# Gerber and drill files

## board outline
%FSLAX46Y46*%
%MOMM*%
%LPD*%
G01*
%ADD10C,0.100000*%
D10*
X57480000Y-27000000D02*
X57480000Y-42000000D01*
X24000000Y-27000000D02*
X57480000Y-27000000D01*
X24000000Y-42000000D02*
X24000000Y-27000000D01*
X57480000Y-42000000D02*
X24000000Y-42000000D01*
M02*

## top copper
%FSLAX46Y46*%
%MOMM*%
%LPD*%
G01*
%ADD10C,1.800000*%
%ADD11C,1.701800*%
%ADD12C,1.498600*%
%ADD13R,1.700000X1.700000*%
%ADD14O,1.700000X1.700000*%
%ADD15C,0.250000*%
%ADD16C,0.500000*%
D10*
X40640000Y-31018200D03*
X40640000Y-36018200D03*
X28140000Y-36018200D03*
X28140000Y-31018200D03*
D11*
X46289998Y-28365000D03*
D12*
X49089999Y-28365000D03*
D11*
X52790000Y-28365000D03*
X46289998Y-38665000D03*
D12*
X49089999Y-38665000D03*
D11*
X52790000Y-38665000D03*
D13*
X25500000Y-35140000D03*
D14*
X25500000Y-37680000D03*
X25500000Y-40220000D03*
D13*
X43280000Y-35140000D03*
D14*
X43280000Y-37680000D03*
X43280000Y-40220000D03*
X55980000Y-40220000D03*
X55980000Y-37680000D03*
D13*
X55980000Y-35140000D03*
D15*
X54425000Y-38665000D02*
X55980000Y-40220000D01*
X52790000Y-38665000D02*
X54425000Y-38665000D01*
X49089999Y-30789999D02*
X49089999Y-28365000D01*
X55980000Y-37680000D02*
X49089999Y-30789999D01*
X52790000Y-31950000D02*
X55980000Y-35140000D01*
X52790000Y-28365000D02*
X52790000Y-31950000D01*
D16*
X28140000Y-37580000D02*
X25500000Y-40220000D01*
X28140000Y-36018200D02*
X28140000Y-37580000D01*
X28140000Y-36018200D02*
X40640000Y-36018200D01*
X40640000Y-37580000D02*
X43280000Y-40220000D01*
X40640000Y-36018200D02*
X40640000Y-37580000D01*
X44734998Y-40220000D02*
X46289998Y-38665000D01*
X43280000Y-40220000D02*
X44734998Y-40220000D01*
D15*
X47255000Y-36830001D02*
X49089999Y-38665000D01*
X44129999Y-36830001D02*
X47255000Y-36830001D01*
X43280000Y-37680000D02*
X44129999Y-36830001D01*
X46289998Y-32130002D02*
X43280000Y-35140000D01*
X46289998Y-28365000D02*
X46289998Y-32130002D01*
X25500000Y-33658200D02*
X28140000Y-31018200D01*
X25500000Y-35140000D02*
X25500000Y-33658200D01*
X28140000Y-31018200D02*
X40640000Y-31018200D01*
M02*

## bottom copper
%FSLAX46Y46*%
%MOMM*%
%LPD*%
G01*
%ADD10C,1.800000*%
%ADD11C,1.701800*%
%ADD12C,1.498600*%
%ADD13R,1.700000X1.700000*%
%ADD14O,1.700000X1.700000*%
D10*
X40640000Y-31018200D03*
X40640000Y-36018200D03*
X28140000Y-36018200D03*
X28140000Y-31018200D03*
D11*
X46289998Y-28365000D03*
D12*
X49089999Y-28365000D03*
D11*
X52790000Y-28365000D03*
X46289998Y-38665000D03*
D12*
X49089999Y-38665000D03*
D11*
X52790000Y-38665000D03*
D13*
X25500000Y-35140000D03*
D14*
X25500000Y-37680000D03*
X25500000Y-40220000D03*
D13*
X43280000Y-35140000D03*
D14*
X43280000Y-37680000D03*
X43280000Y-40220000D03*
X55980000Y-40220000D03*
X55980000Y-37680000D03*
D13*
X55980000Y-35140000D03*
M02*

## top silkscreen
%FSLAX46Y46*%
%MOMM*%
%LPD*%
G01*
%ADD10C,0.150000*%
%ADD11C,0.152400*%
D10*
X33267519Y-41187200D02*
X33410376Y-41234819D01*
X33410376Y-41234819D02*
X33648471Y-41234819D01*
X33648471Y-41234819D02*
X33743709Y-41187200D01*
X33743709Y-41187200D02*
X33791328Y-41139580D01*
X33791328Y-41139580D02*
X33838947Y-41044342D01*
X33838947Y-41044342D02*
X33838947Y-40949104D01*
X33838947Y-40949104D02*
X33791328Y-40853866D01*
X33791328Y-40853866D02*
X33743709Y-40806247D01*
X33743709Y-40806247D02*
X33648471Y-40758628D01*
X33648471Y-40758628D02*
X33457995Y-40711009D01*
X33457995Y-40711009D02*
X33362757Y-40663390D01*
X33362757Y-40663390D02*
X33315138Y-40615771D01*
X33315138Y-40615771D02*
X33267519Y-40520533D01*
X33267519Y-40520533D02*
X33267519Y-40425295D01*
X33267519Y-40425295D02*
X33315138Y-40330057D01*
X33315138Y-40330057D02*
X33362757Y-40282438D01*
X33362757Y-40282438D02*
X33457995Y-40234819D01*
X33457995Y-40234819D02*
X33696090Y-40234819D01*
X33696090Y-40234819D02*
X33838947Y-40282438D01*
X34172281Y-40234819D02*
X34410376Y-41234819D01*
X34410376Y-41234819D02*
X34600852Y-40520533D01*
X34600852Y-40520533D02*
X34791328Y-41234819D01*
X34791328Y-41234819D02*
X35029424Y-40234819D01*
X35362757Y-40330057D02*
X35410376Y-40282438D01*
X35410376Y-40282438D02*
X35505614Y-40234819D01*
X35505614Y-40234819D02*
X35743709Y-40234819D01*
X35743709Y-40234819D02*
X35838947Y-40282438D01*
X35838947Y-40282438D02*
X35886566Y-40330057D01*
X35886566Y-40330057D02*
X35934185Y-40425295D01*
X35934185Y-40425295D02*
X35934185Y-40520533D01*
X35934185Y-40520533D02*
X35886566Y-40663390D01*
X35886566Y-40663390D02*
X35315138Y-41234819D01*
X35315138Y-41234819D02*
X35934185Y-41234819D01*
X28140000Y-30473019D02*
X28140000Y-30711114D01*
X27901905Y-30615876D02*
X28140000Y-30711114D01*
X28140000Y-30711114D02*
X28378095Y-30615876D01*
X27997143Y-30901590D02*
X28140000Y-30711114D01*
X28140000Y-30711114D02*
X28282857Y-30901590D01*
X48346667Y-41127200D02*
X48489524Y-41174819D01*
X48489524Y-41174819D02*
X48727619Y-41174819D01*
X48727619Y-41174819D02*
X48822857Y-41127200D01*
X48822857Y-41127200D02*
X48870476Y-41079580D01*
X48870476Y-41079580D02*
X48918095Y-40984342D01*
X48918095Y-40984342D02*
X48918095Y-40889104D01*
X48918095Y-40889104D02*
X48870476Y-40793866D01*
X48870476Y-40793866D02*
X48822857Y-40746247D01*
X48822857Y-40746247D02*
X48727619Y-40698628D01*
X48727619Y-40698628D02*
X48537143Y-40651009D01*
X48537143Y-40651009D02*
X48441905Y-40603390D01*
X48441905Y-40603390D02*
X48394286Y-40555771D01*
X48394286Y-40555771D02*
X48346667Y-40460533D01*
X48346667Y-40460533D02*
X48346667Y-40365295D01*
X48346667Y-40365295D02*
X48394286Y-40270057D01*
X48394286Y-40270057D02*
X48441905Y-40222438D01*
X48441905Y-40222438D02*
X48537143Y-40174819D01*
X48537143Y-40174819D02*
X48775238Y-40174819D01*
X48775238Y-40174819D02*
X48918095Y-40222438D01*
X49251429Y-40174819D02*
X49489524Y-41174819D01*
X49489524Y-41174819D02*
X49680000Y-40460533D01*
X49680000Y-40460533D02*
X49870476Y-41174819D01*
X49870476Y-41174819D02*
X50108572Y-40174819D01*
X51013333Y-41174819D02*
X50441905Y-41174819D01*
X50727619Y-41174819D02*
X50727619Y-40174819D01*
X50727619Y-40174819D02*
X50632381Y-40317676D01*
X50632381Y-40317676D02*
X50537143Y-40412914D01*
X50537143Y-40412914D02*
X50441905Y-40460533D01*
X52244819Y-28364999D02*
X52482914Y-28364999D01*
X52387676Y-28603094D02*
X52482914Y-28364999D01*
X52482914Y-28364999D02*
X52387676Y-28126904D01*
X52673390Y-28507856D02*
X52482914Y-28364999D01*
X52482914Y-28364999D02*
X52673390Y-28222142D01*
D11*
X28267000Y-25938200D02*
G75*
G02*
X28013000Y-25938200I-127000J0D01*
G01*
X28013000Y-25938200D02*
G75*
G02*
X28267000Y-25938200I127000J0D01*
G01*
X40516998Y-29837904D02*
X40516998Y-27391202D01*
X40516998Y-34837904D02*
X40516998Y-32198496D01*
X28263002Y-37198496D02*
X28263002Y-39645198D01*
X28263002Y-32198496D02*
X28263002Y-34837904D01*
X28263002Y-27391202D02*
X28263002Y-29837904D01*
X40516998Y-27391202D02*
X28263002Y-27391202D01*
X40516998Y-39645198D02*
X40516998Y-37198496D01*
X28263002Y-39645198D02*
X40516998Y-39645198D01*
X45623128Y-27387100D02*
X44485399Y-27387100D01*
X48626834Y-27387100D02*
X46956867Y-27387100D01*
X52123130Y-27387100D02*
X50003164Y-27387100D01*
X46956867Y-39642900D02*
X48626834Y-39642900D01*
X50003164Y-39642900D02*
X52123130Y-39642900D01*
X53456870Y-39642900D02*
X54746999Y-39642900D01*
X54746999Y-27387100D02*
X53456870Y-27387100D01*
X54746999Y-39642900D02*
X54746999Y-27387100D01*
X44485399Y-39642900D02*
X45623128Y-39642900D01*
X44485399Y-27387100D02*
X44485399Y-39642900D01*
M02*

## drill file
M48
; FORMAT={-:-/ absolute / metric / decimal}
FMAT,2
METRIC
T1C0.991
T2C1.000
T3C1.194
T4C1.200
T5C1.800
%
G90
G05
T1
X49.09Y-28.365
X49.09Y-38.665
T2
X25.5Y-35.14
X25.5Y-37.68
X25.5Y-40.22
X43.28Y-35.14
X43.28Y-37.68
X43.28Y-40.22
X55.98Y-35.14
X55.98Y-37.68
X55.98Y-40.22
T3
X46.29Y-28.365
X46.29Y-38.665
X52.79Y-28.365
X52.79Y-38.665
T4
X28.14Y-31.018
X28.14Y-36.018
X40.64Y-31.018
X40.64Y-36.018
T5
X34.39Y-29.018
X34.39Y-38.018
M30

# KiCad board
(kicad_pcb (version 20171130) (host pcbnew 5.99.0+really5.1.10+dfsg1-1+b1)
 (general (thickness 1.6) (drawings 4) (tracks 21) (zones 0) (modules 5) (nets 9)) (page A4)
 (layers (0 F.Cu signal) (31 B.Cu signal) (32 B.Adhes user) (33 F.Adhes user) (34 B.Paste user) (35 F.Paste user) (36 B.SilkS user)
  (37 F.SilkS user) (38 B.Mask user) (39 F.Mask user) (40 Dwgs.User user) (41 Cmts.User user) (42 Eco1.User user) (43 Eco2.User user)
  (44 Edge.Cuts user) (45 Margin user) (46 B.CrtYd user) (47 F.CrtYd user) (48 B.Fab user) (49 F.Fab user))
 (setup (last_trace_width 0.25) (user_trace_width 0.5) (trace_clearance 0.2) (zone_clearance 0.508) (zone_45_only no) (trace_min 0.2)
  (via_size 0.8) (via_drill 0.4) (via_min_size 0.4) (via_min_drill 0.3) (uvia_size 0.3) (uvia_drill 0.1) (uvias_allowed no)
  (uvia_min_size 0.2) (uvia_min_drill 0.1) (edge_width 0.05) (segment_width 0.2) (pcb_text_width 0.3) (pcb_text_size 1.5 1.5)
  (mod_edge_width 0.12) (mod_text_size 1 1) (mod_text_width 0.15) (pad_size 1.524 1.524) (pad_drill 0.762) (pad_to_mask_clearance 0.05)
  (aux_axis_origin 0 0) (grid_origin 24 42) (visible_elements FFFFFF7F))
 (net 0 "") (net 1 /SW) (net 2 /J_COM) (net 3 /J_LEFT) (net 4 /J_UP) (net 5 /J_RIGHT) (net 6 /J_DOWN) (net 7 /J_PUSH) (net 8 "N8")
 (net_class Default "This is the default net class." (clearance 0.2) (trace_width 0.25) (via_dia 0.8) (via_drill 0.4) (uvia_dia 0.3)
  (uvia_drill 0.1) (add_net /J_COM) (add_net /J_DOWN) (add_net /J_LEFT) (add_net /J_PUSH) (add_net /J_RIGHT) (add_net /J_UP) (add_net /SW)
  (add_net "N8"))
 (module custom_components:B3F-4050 (layer F.Cu) (at 28.14 31.0182)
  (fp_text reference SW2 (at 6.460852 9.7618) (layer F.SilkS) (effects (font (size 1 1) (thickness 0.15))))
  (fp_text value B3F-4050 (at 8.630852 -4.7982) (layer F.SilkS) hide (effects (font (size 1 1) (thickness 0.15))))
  (fp_circle (center 0 -5.08) (end 0.127 -5.08) (layer F.SilkS) (width 0.1524))
  (fp_line (start 12.376998 -1.180296) (end 12.376998 -3.626998) (layer F.SilkS) (width 0.1524))
  (fp_line (start 12.376998 3.819704) (end 12.376998 1.180296) (layer F.SilkS) (width 0.1524))
  (fp_line (start 0.123002 6.180296) (end 0.123002 8.626998) (layer F.SilkS) (width 0.1524))
  (fp_line (start 0.123002 1.180296) (end 0.123002 3.819704) (layer F.SilkS) (width 0.1524))
  (fp_line (start 0.123002 -3.626998) (end 0.123002 -1.180296) (layer F.SilkS) (width 0.1524))
  (fp_line (start 12.376998 -3.626998) (end 0.123002 -3.626998) (layer F.SilkS) (width 0.1524))
  (fp_line (start 12.376998 8.626998) (end 12.376998 6.180296) (layer F.SilkS) (width 0.1524))
  (fp_line (start 0.123002 8.626998) (end 12.376998 8.626998) (layer F.SilkS) (width 0.1524))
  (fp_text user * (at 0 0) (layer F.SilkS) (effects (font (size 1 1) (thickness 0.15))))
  (pad "" np_thru_hole circle (at 6.25 7) (size 1.8 1.8) (drill 1.8) (layers *.Cu *.Mask))
  (pad "" np_thru_hole circle (at 6.25 -2) (size 1.8 1.8) (drill 1.8) (layers *.Cu *.Mask))
  (pad 2 thru_hole circle (at 12.5 0) (size 1.8 1.8) (drill 1.2) (layers *.Cu *.Mask) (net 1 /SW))
  (pad 4 thru_hole circle (at 12.5 5) (size 1.8 1.8) (drill 1.2) (layers *.Cu *.Mask) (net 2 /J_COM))
  (pad 3 thru_hole circle (at 0 5) (size 1.8 1.8) (drill 1.2) (layers *.Cu *.Mask) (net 2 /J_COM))
  (pad 1 thru_hole circle (at 0 0) (size 1.8 1.8) (drill 1.2) (layers *.Cu *.Mask) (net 1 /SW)))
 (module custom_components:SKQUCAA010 (layer F.Cu) (at 52.79 28.365 270)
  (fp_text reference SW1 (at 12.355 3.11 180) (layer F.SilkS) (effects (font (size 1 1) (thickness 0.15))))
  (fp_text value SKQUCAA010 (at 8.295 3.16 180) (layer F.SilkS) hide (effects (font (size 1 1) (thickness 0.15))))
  (fp_line (start -0.9779 7.166872) (end -0.9779 8.304601) (layer F.SilkS) (width 0.1524))
  (fp_line (start -0.9779 4.163166) (end -0.9779 5.833133) (layer F.SilkS) (width 0.1524))
  (fp_line (start -0.9779 0.66687) (end -0.9779 2.786836) (layer F.SilkS) (width 0.1524))
  (fp_line (start 11.2779 5.833133) (end 11.2779 4.163166) (layer F.SilkS) (width 0.1524))
  (fp_line (start 11.2779 2.786836) (end 11.2779 0.66687) (layer F.SilkS) (width 0.1524))
  (fp_line (start 11.2779 -0.66687) (end 11.2779 -1.956999) (layer F.SilkS) (width 0.1524))
  (fp_line (start -0.9779 -1.956999) (end -0.9779 -0.66687) (layer F.SilkS) (width 0.1524))
  (fp_line (start 11.2779 -1.956999) (end -0.9779 -1.956999) (layer F.SilkS) (width 0.1524))
  (fp_line (start 11.2779 8.304601) (end 11.2779 7.166872) (layer F.SilkS) (width 0.1524))
  (fp_line (start -0.9779 8.304601) (end 11.2779 8.304601) (layer F.SilkS) (width 0.1524))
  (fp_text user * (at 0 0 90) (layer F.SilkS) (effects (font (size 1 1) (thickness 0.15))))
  (pad 3 thru_hole circle (at 0 6.500002 270) (size 1.7018 1.7018) (drill 1.1938) (layers *.Cu *.Mask) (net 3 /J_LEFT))
  (pad 2 thru_hole circle (at 0 3.700001 270) (size 1.4986 1.4986) (drill 0.9906) (layers *.Cu *.Mask) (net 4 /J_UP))
  (pad 1 thru_hole circle (at 0 0 270) (size 1.7018 1.7018) (drill 1.1938) (layers *.Cu *.Mask) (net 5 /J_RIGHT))
  (pad 4 thru_hole circle (at 10.3 6.500002 270) (size 1.7018 1.7018) (drill 1.1938) (layers *.Cu *.Mask) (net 2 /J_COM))
  (pad 5 thru_hole circle (at 10.3 3.700001 270) (size 1.4986 1.4986) (drill 0.9906) (layers *.Cu *.Mask) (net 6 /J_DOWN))
  (pad 6 thru_hole circle (at 10.3 0 270) (size 1.7018 1.7018) (drill 1.1938) (layers *.Cu *.Mask) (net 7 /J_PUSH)))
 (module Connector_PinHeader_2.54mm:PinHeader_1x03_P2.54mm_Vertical (layer B.Cu) (at 25.5 35.14 180)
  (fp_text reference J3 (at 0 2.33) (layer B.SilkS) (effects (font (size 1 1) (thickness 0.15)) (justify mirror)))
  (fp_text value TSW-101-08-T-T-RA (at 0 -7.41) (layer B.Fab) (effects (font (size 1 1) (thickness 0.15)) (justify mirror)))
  (pad 1 thru_hole rect (at 0 0 180) (size 1.7 1.7) (drill 1) (layers *.Cu *.Mask) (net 1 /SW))
  (pad 2 thru_hole oval (at 0 -2.54 180) (size 1.7 1.7) (drill 1) (layers *.Cu *.Mask) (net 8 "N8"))
  (pad 3 thru_hole oval (at 0 -5.08 180) (size 1.7 1.7) (drill 1) (layers *.Cu *.Mask) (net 2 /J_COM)))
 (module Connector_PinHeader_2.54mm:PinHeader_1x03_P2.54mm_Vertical (layer B.Cu) (at 43.28 35.14 180)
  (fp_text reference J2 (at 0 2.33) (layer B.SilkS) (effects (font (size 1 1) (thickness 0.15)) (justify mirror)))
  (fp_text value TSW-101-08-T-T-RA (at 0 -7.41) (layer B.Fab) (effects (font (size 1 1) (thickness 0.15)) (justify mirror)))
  (pad 1 thru_hole rect (at 0 0 180) (size 1.7 1.7) (drill 1) (layers *.Cu *.Mask) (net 3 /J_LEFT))
  (pad 2 thru_hole oval (at 0 -2.54 180) (size 1.7 1.7) (drill 1) (layers *.Cu *.Mask) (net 6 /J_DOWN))
  (pad 3 thru_hole oval (at 0 -5.08 180) (size 1.7 1.7) (drill 1) (layers *.Cu *.Mask) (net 2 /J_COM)))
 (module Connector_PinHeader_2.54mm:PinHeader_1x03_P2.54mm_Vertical (layer B.Cu) (at 55.98 35.14 180)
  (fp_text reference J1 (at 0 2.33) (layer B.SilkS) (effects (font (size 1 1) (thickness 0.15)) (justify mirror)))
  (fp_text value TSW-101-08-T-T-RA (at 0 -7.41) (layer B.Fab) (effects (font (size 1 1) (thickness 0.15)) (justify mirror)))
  (pad 3 thru_hole oval (at 0 -5.08 180) (size 1.7 1.7) (drill 1) (layers *.Cu *.Mask) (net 7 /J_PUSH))
  (pad 2 thru_hole oval (at 0 -2.54 180) (size 1.7 1.7) (drill 1) (layers *.Cu *.Mask) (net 4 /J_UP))
  (pad 1 thru_hole rect (at 0 0 180) (size 1.7 1.7) (drill 1) (layers *.Cu *.Mask) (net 5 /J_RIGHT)))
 (gr_line (start 57.48 27) (end 57.48 42) (layer Edge.Cuts) (width 0.1))
 (gr_line (start 24 27) (end 57.48 27) (layer Edge.Cuts) (width 0.1))
 (gr_line (start 24 42) (end 24 27) (layer Edge.Cuts) (width 0.1))
 (gr_line (start 57.48 42) (end 24 42) (layer Edge.Cuts) (width 0.1))
 (segment (start 54.425 38.665) (end 55.98 40.22) (width 0.25) (layer F.Cu) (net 7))
 (segment (start 52.79 38.665) (end 54.425 38.665) (width 0.25) (layer F.Cu) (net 7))
 (segment (start 49.089999 30.789999) (end 49.089999 28.365) (width 0.25) (layer F.Cu) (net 4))
 (segment (start 55.98 37.68) (end 49.089999 30.789999) (width 0.25) (layer F.Cu) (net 4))
 (segment (start 52.79 31.95) (end 55.98 35.14) (width 0.25) (layer F.Cu) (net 5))
 (segment (start 52.79 28.365) (end 52.79 31.95) (width 0.25) (layer F.Cu) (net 5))
 (segment (start 28.14 37.58) (end 25.5 40.22) (width 0.5) (layer F.Cu) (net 2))
 (segment (start 28.14 36.0182) (end 28.14 37.58) (width 0.5) (layer F.Cu) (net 2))
 (segment (start 28.14 36.0182) (end 40.64 36.0182) (width 0.5) (layer F.Cu) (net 2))
 (segment (start 40.64 37.58) (end 43.28 40.22) (width 0.5) (layer F.Cu) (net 2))
 (segment (start 40.64 36.0182) (end 40.64 37.58) (width 0.5) (layer F.Cu) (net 2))
 (segment (start 44.734998 40.22) (end 46.289998 38.665) (width 0.5) (layer F.Cu) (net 2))
 (segment (start 43.28 40.22) (end 44.734998 40.22) (width 0.5) (layer F.Cu) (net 2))
 (segment (start 47.255 36.830001) (end 49.089999 38.665) (width 0.25) (layer F.Cu) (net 6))
 (segment (start 44.129999 36.830001) (end 47.255 36.830001) (width 0.25) (layer F.Cu) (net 6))
 (segment (start 43.28 37.68) (end 44.129999 36.830001) (width 0.25) (layer F.Cu) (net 6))
 (segment (start 46.289998 32.130002) (end 43.28 35.14) (width 0.25) (layer F.Cu) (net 3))
 (segment (start 46.289998 28.365) (end 46.289998 32.130002) (width 0.25) (layer F.Cu) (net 3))
 (segment (start 25.5 33.6582) (end 28.14 31.0182) (width 0.25) (layer F.Cu) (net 1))
 (segment (start 25.5 35.14) (end 25.5 33.6582) (width 0.25) (layer F.Cu) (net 1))
 (segment (start 28.14 31.0182) (end 40.64 31.0182) (width 0.25) (layer F.Cu) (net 1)))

